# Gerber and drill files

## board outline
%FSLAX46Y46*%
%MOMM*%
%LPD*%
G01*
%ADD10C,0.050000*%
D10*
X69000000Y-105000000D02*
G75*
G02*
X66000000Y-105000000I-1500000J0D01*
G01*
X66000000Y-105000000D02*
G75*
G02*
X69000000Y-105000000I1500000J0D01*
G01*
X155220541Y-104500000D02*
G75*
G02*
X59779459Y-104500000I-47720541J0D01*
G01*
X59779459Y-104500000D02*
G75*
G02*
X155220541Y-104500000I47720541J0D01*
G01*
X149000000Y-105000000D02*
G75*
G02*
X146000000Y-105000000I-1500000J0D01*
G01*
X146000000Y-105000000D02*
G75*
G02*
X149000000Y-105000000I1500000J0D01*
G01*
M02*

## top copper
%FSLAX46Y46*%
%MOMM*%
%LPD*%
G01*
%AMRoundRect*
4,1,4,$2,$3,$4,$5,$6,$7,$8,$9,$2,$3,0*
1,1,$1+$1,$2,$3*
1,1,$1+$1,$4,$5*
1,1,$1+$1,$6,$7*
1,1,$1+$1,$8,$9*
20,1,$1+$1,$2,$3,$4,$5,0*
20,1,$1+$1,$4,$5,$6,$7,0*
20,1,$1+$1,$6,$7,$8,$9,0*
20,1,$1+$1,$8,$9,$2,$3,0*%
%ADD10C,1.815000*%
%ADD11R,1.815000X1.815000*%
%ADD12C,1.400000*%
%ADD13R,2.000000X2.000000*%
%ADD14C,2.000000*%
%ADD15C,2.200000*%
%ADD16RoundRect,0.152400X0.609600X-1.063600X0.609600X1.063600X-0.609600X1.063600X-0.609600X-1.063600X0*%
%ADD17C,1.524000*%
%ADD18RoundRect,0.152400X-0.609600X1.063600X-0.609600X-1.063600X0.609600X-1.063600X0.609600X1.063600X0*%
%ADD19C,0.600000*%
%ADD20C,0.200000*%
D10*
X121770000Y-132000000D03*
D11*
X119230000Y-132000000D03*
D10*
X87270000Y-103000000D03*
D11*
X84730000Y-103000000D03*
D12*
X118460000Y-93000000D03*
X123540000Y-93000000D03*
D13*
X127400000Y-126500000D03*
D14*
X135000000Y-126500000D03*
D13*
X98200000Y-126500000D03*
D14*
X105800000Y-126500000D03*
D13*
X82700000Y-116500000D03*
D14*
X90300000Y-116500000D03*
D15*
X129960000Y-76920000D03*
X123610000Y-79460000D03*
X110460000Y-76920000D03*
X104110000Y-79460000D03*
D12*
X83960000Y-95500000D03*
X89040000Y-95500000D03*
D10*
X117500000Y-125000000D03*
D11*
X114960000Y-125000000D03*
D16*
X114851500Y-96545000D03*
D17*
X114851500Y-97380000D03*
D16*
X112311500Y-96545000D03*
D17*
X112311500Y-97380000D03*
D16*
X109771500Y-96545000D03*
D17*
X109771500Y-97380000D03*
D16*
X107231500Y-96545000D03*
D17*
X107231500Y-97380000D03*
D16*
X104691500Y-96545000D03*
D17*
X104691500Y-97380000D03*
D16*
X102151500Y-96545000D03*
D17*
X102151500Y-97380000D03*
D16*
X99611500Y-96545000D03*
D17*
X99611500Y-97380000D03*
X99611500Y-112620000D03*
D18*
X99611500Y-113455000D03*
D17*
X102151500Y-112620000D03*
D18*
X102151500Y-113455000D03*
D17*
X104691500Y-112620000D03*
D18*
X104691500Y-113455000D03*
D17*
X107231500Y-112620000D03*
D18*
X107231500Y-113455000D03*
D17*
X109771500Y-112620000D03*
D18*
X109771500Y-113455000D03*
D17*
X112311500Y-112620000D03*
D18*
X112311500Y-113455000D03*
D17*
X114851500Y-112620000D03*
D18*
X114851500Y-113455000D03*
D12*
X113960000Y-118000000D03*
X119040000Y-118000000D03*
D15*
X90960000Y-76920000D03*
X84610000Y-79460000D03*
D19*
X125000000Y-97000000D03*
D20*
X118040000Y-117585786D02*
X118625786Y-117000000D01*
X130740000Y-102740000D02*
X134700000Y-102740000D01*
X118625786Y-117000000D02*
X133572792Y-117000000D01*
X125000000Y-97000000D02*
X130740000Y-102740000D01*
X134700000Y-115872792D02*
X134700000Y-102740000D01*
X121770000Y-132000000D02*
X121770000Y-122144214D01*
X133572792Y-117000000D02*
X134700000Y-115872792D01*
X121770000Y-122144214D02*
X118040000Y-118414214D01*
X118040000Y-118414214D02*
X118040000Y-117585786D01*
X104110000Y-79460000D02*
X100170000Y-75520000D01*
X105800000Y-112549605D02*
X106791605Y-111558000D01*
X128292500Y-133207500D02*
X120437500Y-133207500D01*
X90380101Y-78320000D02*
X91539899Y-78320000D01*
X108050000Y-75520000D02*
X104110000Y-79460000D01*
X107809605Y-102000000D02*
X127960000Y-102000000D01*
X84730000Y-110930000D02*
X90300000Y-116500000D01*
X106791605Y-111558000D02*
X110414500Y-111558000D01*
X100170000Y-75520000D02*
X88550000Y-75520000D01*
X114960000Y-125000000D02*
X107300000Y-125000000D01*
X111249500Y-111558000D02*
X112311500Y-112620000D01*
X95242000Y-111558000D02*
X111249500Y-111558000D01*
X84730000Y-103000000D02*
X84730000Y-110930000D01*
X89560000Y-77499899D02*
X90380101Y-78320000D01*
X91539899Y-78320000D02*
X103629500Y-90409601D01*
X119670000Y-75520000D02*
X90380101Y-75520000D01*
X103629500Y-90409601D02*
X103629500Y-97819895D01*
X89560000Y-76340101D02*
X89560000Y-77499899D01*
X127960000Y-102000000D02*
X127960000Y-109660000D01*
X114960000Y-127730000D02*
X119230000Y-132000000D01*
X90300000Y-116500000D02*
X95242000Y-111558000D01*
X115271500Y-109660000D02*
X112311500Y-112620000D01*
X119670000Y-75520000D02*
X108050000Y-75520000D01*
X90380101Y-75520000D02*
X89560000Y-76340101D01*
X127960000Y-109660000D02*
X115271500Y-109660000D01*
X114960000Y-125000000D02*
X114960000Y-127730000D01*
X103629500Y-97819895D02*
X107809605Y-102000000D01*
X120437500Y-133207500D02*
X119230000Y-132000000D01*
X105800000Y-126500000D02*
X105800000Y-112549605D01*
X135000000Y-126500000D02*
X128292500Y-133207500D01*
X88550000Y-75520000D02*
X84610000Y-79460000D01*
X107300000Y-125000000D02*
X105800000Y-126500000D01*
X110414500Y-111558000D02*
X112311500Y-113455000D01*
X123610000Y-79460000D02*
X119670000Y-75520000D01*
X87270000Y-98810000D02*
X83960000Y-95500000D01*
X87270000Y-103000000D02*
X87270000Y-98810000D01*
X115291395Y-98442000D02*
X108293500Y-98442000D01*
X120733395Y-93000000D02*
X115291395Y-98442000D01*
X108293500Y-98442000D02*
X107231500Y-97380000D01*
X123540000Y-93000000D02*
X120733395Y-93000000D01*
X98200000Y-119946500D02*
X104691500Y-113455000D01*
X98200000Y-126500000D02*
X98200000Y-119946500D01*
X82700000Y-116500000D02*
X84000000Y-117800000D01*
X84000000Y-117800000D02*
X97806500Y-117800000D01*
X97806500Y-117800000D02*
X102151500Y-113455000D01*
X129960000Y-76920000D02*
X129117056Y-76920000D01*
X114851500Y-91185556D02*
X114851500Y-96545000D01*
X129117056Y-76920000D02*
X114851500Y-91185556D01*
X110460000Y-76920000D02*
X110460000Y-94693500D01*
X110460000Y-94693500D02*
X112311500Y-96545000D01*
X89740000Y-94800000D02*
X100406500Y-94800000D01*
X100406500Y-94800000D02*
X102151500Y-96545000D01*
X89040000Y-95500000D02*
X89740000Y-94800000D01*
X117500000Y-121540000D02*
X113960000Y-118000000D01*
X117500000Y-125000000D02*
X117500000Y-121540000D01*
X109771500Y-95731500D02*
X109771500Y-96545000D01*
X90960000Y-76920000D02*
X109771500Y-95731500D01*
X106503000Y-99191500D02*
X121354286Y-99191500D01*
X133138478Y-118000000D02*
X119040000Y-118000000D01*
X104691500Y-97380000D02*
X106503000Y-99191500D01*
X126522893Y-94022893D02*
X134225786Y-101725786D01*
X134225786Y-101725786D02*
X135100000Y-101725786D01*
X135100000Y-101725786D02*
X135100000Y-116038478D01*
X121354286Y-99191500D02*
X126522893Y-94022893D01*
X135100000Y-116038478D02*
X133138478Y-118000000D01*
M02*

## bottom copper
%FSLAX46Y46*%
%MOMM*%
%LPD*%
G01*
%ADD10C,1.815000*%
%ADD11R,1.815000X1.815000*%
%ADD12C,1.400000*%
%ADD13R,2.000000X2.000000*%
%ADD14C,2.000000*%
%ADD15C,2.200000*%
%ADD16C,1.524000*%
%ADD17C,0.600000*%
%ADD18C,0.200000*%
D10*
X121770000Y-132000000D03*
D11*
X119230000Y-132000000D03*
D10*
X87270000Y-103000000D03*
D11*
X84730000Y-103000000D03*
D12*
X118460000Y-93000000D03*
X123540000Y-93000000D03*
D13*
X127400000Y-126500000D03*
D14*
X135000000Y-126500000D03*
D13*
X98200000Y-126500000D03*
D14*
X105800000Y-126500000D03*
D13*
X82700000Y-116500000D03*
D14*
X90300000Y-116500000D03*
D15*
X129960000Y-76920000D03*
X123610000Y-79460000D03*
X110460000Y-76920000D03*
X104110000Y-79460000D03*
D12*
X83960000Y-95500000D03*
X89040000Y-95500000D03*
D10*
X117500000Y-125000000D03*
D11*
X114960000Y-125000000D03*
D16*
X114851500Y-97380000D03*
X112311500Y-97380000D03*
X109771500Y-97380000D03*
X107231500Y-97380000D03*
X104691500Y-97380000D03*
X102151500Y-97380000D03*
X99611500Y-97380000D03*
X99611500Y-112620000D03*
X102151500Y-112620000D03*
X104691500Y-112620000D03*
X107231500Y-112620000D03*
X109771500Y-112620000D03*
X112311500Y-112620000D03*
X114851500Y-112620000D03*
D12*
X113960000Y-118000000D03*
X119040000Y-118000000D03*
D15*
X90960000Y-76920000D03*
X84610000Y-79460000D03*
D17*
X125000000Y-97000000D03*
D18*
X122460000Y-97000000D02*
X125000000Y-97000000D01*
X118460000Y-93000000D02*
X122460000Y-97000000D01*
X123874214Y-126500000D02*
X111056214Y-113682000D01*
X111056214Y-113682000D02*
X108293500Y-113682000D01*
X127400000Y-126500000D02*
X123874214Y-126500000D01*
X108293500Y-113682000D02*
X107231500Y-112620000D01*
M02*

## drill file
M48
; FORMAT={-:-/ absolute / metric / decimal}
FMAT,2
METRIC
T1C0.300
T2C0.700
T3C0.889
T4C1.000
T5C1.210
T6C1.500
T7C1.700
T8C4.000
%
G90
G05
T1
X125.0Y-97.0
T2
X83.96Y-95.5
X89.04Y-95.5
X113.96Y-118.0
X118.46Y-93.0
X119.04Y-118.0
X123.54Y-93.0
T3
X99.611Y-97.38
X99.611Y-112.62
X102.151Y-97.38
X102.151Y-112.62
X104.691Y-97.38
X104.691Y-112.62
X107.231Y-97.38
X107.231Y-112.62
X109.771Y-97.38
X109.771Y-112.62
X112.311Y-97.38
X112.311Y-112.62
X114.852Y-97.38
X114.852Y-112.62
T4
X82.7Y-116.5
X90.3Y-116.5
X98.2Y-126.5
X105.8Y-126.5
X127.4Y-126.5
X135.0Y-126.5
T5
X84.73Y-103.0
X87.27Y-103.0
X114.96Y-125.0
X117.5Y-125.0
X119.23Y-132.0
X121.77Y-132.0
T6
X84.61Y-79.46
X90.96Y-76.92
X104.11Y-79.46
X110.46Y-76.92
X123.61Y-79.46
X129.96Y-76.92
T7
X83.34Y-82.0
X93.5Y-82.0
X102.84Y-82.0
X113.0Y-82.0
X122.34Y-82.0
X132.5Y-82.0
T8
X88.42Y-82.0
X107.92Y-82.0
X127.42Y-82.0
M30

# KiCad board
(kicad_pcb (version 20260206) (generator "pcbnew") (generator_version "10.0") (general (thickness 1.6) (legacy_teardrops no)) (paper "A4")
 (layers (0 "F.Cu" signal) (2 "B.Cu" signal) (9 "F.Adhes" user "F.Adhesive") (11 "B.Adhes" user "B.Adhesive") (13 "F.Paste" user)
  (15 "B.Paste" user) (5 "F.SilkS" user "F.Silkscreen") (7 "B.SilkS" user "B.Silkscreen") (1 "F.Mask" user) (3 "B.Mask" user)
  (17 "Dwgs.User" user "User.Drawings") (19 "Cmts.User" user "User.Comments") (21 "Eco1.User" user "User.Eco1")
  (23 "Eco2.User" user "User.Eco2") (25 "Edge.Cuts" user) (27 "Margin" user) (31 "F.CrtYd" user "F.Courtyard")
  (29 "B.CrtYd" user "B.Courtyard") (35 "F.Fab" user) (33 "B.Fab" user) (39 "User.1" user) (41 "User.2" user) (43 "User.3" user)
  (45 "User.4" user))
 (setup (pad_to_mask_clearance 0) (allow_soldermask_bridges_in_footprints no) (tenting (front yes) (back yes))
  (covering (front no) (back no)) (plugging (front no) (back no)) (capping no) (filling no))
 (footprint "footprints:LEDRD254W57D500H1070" (layer "F.Cu") (at 120.5 132)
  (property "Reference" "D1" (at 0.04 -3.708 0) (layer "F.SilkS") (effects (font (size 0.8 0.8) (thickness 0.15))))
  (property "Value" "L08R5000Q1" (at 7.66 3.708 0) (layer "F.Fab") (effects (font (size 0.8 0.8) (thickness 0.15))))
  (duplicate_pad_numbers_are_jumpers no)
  (pad "A" thru_hole circle (at 1.27 0) (size 1.815 1.815) (drill 1.21) (layers "*.Cu" "*.Mask") (remove_unused_layers no)
   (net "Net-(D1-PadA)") (solder_mask_margin 0.102))
  (pad "C" thru_hole rect (at -1.27 0) (size 1.815 1.815) (drill 1.21) (layers "*.Cu" "*.Mask") (remove_unused_layers no) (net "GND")
   (solder_mask_margin 0.102)))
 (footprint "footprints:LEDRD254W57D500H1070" (layer "F.Cu") (at 86 103)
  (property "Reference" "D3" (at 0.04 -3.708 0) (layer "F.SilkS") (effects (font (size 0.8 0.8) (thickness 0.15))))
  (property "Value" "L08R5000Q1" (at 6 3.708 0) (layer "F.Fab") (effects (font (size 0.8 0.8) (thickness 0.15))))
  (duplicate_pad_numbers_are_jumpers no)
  (pad "A" thru_hole circle (at 1.27 0) (size 1.815 1.815) (drill 1.21) (layers "*.Cu" "*.Mask") (remove_unused_layers no)
   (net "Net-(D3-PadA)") (solder_mask_margin 0.102))
  (pad "C" thru_hole rect (at -1.27 0) (size 1.815 1.815) (drill 1.21) (layers "*.Cu" "*.Mask") (remove_unused_layers no) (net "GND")
   (solder_mask_margin 0.102)))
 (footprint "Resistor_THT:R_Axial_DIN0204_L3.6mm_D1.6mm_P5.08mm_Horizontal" (layer "F.Cu") (at 118.46 93)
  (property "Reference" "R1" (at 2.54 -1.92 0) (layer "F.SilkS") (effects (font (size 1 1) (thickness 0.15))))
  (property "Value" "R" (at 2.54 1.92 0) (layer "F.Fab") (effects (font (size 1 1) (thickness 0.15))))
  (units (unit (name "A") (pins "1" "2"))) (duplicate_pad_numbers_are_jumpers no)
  (pad "1" thru_hole circle (at 0 0) (size 1.4 1.4) (drill 0.7) (layers "*.Cu" "*.Mask") (remove_unused_layers no) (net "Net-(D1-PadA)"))
  (pad "2" thru_hole circle (at 5.08 0) (size 1.4 1.4) (drill 0.7) (layers "*.Cu" "*.Mask") (remove_unused_layers no)
   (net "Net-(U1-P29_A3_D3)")))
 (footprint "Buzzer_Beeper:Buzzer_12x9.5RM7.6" (layer "F.Cu") (at 127.4 126.5)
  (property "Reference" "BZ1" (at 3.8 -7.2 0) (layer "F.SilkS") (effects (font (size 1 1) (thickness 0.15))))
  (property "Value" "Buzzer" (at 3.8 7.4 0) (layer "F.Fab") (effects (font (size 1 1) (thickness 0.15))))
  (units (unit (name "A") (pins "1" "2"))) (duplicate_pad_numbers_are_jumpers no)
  (pad "1" thru_hole rect (at 0 0) (size 2 2) (drill 1) (layers "*.Cu" "*.Mask") (remove_unused_layers no) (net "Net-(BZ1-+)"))
  (pad "2" thru_hole circle (at 7.6 0) (size 2 2) (drill 1) (layers "*.Cu" "*.Mask") (remove_unused_layers no) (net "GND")))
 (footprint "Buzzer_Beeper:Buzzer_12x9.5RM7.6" (layer "F.Cu") (at 98.2 126.5)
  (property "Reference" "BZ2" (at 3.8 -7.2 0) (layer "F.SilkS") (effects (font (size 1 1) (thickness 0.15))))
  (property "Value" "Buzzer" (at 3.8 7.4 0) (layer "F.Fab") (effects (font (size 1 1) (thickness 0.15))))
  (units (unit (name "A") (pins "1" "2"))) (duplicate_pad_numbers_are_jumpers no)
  (pad "1" thru_hole rect (at 0 0) (size 2 2) (drill 1) (layers "*.Cu" "*.Mask") (remove_unused_layers no) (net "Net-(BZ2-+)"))
  (pad "2" thru_hole circle (at 7.6 0) (size 2 2) (drill 1) (layers "*.Cu" "*.Mask") (remove_unused_layers no) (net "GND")))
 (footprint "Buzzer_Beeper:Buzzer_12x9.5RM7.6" (layer "F.Cu") (at 82.7 116.5)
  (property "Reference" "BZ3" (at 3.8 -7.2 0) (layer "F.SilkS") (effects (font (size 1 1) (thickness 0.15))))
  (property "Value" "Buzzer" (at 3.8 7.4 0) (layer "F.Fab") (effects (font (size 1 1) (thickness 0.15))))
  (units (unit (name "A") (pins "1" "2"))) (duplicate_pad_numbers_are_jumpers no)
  (pad "1" thru_hole rect (at 0 0) (size 2 2) (drill 1) (layers "*.Cu" "*.Mask") (remove_unused_layers no) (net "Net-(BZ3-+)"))
  (pad "2" thru_hole circle (at 7.6 0) (size 2 2) (drill 1) (layers "*.Cu" "*.Mask") (remove_unused_layers no) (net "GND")))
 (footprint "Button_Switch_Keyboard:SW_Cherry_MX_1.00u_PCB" (layer "F.Cu") (at 129.96 76.92)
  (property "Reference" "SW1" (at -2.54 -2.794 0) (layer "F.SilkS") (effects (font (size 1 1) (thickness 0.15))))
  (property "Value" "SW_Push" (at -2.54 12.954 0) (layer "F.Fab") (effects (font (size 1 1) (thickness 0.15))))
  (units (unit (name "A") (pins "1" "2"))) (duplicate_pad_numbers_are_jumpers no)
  (pad "" np_thru_hole circle (at -7.62 5.08) (size 1.7 1.7) (drill 1.7) (layers "*.Cu" "*.Mask"))
  (pad "" np_thru_hole circle (at -2.54 5.08) (size 4 4) (drill 4) (layers "*.Cu" "*.Mask"))
  (pad "" np_thru_hole circle (at 2.54 5.08) (size 1.7 1.7) (drill 1.7) (layers "*.Cu" "*.Mask"))
  (pad "1" thru_hole circle (at 0 0) (size 2.2 2.2) (drill 1.5) (layers "*.Cu" "*.Mask") (remove_unused_layers no)
   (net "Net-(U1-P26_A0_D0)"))
  (pad "2" thru_hole circle (at -6.35 2.54) (size 2.2 2.2) (drill 1.5) (layers "*.Cu" "*.Mask") (remove_unused_layers no) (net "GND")))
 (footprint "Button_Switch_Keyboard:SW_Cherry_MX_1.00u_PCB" (layer "F.Cu") (at 110.46 76.92)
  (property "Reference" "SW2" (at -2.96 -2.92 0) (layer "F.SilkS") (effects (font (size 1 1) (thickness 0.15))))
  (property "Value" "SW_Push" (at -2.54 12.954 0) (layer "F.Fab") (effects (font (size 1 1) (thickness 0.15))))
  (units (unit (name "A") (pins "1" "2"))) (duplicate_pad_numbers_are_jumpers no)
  (pad "" np_thru_hole circle (at -7.62 5.08) (size 1.7 1.7) (drill 1.7) (layers "*.Cu" "*.Mask"))
  (pad "" np_thru_hole circle (at -2.54 5.08) (size 4 4) (drill 4) (layers "*.Cu" "*.Mask"))
  (pad "" np_thru_hole circle (at 2.54 5.08) (size 1.7 1.7) (drill 1.7) (layers "*.Cu" "*.Mask"))
  (pad "1" thru_hole circle (at 0 0) (size 2.2 2.2) (drill 1.5) (layers "*.Cu" "*.Mask") (remove_unused_layers no)
   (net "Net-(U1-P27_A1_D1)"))
  (pad "2" thru_hole circle (at -6.35 2.54) (size 2.2 2.2) (drill 1.5) (layers "*.Cu" "*.Mask") (remove_unused_layers no) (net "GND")))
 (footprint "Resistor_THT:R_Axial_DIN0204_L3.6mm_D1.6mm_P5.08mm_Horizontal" (layer "F.Cu") (at 83.96 95.5)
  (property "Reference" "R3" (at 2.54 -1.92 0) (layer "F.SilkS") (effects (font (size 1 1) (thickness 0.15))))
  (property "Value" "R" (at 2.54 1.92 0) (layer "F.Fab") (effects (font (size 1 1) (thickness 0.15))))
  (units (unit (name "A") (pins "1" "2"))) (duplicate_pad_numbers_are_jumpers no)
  (pad "1" thru_hole circle (at 0 0) (size 1.4 1.4) (drill 0.7) (layers "*.Cu" "*.Mask") (remove_unused_layers no) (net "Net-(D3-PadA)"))
  (pad "2" thru_hole circle (at 5.08 0) (size 1.4 1.4) (drill 0.7) (layers "*.Cu" "*.Mask") (remove_unused_layers no)
   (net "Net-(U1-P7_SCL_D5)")))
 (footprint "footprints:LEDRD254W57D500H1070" (layer "F.Cu") (at 116.23 125)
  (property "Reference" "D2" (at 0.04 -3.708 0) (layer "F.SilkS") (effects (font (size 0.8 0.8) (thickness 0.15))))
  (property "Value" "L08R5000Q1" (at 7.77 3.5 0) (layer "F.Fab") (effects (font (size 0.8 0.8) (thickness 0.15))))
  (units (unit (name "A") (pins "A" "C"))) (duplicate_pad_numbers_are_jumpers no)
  (pad "A" thru_hole circle (at 1.27 0) (size 1.815 1.815) (drill 1.21) (layers "*.Cu" "*.Mask") (remove_unused_layers no)
   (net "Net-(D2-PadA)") (solder_mask_margin 0.102))
  (pad "C" thru_hole rect (at -1.27 0) (size 1.815 1.815) (drill 1.21) (layers "*.Cu" "*.Mask") (remove_unused_layers no) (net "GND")
   (solder_mask_margin 0.102)))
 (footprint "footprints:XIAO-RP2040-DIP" (layer "F.Cu") (at 107.2315 105)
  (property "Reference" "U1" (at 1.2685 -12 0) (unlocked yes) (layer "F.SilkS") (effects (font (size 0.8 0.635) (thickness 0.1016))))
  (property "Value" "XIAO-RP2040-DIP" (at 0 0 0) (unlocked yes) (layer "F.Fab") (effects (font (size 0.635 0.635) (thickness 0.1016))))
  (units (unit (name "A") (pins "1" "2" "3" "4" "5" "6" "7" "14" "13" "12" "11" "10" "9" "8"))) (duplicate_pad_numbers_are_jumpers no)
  (pad "1" smd roundrect (at 7.62 -8.455 90) (size 2.432 1.524) (layers "F.Cu" "F.Mask") (roundrect_rratio 0.1) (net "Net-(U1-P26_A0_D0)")
   (thermal_bridge_angle 45))
  (pad "1" thru_hole circle (at 7.62 -7.62 90) (size 1.524 1.524) (drill 0.889) (layers "*.Cu" "*.Mask") (remove_unused_layers no)
   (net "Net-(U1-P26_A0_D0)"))
  (pad "2" smd roundrect (at 5.08 -8.455 90) (size 2.432 1.524) (layers "F.Cu" "F.Mask") (roundrect_rratio 0.1) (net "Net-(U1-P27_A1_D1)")
   (thermal_bridge_angle 45))
  (pad "2" thru_hole circle (at 5.08 -7.62 90) (size 1.524 1.524) (drill 0.889) (layers "*.Cu" "*.Mask") (remove_unused_layers no)
   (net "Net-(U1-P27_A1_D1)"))
  (pad "3" smd roundrect (at 2.54 -8.455 90) (size 2.432 1.524) (layers "F.Cu" "F.Mask") (roundrect_rratio 0.1) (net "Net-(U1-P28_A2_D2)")
   (thermal_bridge_angle 45))
  (pad "3" thru_hole circle (at 2.54 -7.62 90) (size 1.524 1.524) (drill 0.889) (layers "*.Cu" "*.Mask") (remove_unused_layers no)
   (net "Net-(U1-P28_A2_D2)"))
  (pad "4" smd roundrect (at 0 -8.455 90) (size 2.432 1.524) (layers "F.Cu" "F.Mask") (roundrect_rratio 0.1) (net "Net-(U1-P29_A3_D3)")
   (thermal_bridge_angle 45))
  (pad "4" thru_hole circle (at 0 -7.62 90) (size 1.524 1.524) (drill 0.889) (layers "*.Cu" "*.Mask") (remove_unused_layers no)
   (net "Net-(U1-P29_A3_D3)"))
  (pad "5" smd roundrect (at -2.54 -8.455 90) (size 2.432 1.524) (layers "F.Cu" "F.Mask") (roundrect_rratio 0.1) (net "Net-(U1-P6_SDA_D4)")
   (thermal_bridge_angle 45))
  (pad "5" thru_hole circle (at -2.54 -7.62 90) (size 1.524 1.524) (drill 0.889) (layers "*.Cu" "*.Mask") (remove_unused_layers no)
   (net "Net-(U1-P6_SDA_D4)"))
  (pad "6" smd roundrect (at -5.08 -8.455 90) (size 2.432 1.524) (layers "F.Cu" "F.Mask") (roundrect_rratio 0.1) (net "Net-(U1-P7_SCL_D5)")
   (thermal_bridge_angle 45))
  (pad "6" thru_hole circle (at -5.08 -7.62 90) (size 1.524 1.524) (drill 0.889) (layers "*.Cu" "*.Mask") (remove_unused_layers no)
   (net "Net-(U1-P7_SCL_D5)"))
  (pad "7" smd roundrect (at -7.62 -8.455 90) (size 2.432 1.524) (layers "F.Cu" "F.Mask") (roundrect_rratio 0.1)
   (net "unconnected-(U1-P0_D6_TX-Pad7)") (thermal_bridge_angle 45))
  (pad "7" thru_hole circle (at -7.62 -7.62 90) (size 1.524 1.524) (drill 0.889) (layers "*.Cu" "*.Mask") (remove_unused_layers no)
   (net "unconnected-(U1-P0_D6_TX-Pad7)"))
  (pad "8" thru_hole circle (at -7.62 7.62 270) (size 1.524 1.524) (drill 0.889) (layers "*.Cu" "*.Mask") (remove_unused_layers no)
   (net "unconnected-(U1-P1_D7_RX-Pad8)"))
  (pad "8" smd roundrect (at -7.62 8.455 270) (size 2.432 1.524) (layers "F.Cu" "F.Mask") (roundrect_rratio 0.1)
   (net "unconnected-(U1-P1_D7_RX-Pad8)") (thermal_bridge_angle 45))
  (pad "9" thru_hole circle (at -5.08 7.62 270) (size 1.524 1.524) (drill 0.889) (layers "*.Cu" "*.Mask") (remove_unused_layers no)
   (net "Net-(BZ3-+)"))
  (pad "9" smd roundrect (at -5.08 8.455 270) (size 2.432 1.524) (layers "F.Cu" "F.Mask") (roundrect_rratio 0.1) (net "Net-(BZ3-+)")
   (thermal_bridge_angle 45))
  (pad "10" thru_hole circle (at -2.54 7.62 270) (size 1.524 1.524) (drill 0.889) (layers "*.Cu" "*.Mask") (remove_unused_layers no)
   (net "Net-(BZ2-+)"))
  (pad "10" smd roundrect (at -2.54 8.455 270) (size 2.432 1.524) (layers "F.Cu" "F.Mask") (roundrect_rratio 0.1) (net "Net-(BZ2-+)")
   (thermal_bridge_angle 45))
  (pad "11" thru_hole circle (at 0 7.62 270) (size 1.524 1.524) (drill 0.889) (layers "*.Cu" "*.Mask") (remove_unused_layers no)
   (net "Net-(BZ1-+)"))
  (pad "11" smd roundrect (at 0 8.455 270) (size 2.432 1.524) (layers "F.Cu" "F.Mask") (roundrect_rratio 0.1) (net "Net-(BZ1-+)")
   (thermal_bridge_angle 45))
  (pad "12" thru_hole circle (at 2.54 7.62 270) (size 1.524 1.524) (drill 0.889) (layers "*.Cu" "*.Mask") (remove_unused_layers no)
   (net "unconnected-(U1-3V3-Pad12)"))
  (pad "12" smd roundrect (at 2.54 8.455 270) (size 2.432 1.524) (layers "F.Cu" "F.Mask") (roundrect_rratio 0.1)
   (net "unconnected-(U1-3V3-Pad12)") (thermal_bridge_angle 45))
  (pad "13" thru_hole circle (at 5.08 7.62 270) (size 1.524 1.524) (drill 0.889) (layers "*.Cu" "*.Mask") (remove_unused_layers no)
   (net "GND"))
  (pad "13" smd roundrect (at 5.08 8.455 270) (size 2.432 1.524) (layers "F.Cu" "F.Mask") (roundrect_rratio 0.1) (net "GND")
   (thermal_bridge_angle 45))
  (pad "14" thru_hole circle (at 7.62 7.62 270) (size 1.524 1.524) (drill 0.889) (layers "*.Cu" "*.Mask") (remove_unused_layers no)
   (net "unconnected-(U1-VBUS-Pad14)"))
  (pad "14" smd roundrect (at 7.62 8.455 270) (size 2.432 1.524) (layers "F.Cu" "F.Mask") (roundrect_rratio 0.1)
   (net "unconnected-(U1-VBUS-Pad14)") (thermal_bridge_angle 45)))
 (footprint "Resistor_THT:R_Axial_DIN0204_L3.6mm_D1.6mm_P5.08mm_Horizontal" (layer "F.Cu") (at 113.96 118)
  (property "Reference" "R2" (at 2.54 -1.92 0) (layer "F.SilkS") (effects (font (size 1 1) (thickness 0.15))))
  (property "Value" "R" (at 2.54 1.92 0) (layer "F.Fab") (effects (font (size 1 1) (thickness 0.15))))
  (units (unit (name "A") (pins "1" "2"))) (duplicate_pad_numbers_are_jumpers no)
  (pad "1" thru_hole circle (at 0 0) (size 1.4 1.4) (drill 0.7) (layers "*.Cu" "*.Mask") (remove_unused_layers no) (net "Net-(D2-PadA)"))
  (pad "2" thru_hole circle (at 5.08 0) (size 1.4 1.4) (drill 0.7) (layers "*.Cu" "*.Mask") (remove_unused_layers no)
   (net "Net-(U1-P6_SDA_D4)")))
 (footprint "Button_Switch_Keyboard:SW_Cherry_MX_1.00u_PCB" (layer "F.Cu") (at 90.96 76.92)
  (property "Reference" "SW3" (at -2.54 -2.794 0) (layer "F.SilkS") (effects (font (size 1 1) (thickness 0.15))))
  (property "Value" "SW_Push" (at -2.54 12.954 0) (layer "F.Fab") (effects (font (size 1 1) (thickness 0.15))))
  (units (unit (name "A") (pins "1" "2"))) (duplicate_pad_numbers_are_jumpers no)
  (pad "" np_thru_hole circle (at -7.62 5.08) (size 1.7 1.7) (drill 1.7) (layers "*.Cu" "*.Mask"))
  (pad "" np_thru_hole circle (at -2.54 5.08) (size 4 4) (drill 4) (layers "*.Cu" "*.Mask"))
  (pad "" np_thru_hole circle (at 2.54 5.08) (size 1.7 1.7) (drill 1.7) (layers "*.Cu" "*.Mask"))
  (pad "1" thru_hole circle (at 0 0) (size 2.2 2.2) (drill 1.5) (layers "*.Cu" "*.Mask") (remove_unused_layers no)
   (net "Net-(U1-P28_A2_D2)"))
  (pad "2" thru_hole circle (at -6.35 2.54) (size 2.2 2.2) (drill 1.5) (layers "*.Cu" "*.Mask") (remove_unused_layers no) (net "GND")))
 (gr_circle (center 67.5 105) (end 66 105) (stroke (width 0.05) (type default)) (fill no) (layer "Edge.Cuts"))
 (gr_circle (center 107.5 104.5) (end 80 65.5) (stroke (width 0.05) (type default)) (fill no) (layer "Edge.Cuts"))
 (gr_circle (center 147.5 105) (end 149 105) (stroke (width 0.05) (type default)) (fill no) (layer "Edge.Cuts"))
 (segment (start 118.04 117.585786) (end 118.625786 117) (width 0.2) (layer "F.Cu") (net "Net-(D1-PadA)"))
 (segment (start 130.74 102.74) (end 134.7 102.74) (width 0.2) (layer "F.Cu") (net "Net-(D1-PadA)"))
 (segment (start 118.625786 117) (end 133.572792 117) (width 0.2) (layer "F.Cu") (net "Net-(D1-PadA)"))
 (segment (start 125 97) (end 130.74 102.74) (width 0.2) (layer "F.Cu") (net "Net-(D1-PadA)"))
 (segment (start 134.7 115.872792) (end 134.7 102.74) (width 0.2) (layer "F.Cu") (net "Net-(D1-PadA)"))
 (segment (start 121.77 132) (end 121.77 122.144214) (width 0.2) (layer "F.Cu") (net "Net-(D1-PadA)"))
 (segment (start 133.572792 117) (end 134.7 115.872792) (width 0.2) (layer "F.Cu") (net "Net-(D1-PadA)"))
 (segment (start 121.77 122.144214) (end 118.04 118.414214) (width 0.2) (layer "F.Cu") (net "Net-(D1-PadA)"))
 (segment (start 118.04 118.414214) (end 118.04 117.585786) (width 0.2) (layer "F.Cu") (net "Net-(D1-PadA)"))
 (via (at 125 97) (size 0.6) (drill 0.3) (layers "F.Cu" "B.Cu") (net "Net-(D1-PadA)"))
 (segment (start 122.46 97) (end 125 97) (width 0.2) (layer "B.Cu") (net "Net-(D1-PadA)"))
 (segment (start 118.46 93) (end 122.46 97) (width 0.2) (layer "B.Cu") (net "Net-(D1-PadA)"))
 (segment (start 104.11 79.46) (end 100.17 75.52) (width 0.2) (layer "F.Cu") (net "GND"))
 (segment (start 105.8 112.549605) (end 106.791605 111.558) (width 0.2) (layer "F.Cu") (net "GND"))
 (segment (start 128.2925 133.2075) (end 120.4375 133.2075) (width 0.2) (layer "F.Cu") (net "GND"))
 (segment (start 90.380101 78.32) (end 91.539899 78.32) (width 0.2) (layer "F.Cu") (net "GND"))
 (segment (start 108.05 75.52) (end 104.11 79.46) (width 0.2) (layer "F.Cu") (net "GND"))
 (segment (start 107.809605 102) (end 127.96 102) (width 0.2) (layer "F.Cu") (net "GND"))
 (segment (start 84.73 110.93) (end 90.3 116.5) (width 0.2) (layer "F.Cu") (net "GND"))
 (segment (start 106.791605 111.558) (end 110.4145 111.558) (width 0.2) (layer "F.Cu") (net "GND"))
 (segment (start 100.17 75.52) (end 88.55 75.52) (width 0.2) (layer "F.Cu") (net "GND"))
 (segment (start 114.96 125) (end 107.3 125) (width 0.2) (layer "F.Cu") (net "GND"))
 (segment (start 111.2495 111.558) (end 112.3115 112.62) (width 0.2) (layer "F.Cu") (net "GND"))
 (segment (start 95.242 111.558) (end 111.2495 111.558) (width 0.2) (layer "F.Cu") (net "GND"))
 (segment (start 84.73 103) (end 84.73 110.93) (width 0.2) (layer "F.Cu") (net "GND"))
 (segment (start 89.56 77.499899) (end 90.380101 78.32) (width 0.2) (layer "F.Cu") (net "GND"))
 (segment (start 91.539899 78.32) (end 103.6295 90.409601) (width 0.2) (layer "F.Cu") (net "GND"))
 (segment (start 119.67 75.52) (end 90.380101 75.52) (width 0.2) (layer "F.Cu") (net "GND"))
 (segment (start 103.6295 90.409601) (end 103.6295 97.819895) (width 0.2) (layer "F.Cu") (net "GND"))
 (segment (start 89.56 76.340101) (end 89.56 77.499899) (width 0.2) (layer "F.Cu") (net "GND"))
 (segment (start 127.96 102) (end 127.96 109.66) (width 0.2) (layer "F.Cu") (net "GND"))
 (segment (start 114.96 127.73) (end 119.23 132) (width 0.2) (layer "F.Cu") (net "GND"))
 (segment (start 90.3 116.5) (end 95.242 111.558) (width 0.2) (layer "F.Cu") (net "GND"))
 (segment (start 115.2715 109.66) (end 112.3115 112.62) (width 0.2) (layer "F.Cu") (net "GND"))
 (segment (start 119.67 75.52) (end 108.05 75.52) (width 0.2) (layer "F.Cu") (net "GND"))
 (segment (start 90.380101 75.52) (end 89.56 76.340101) (width 0.2) (layer "F.Cu") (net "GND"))
 (segment (start 127.96 109.66) (end 115.2715 109.66) (width 0.2) (layer "F.Cu") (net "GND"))
 (segment (start 114.96 125) (end 114.96 127.73) (width 0.2) (layer "F.Cu") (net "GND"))
 (segment (start 103.6295 97.819895) (end 107.809605 102) (width 0.2) (layer "F.Cu") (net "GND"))
 (segment (start 120.4375 133.2075) (end 119.23 132) (width 0.2) (layer "F.Cu") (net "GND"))
 (segment (start 105.8 126.5) (end 105.8 112.549605) (width 0.2) (layer "F.Cu") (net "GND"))
 (segment (start 135 126.5) (end 128.2925 133.2075) (width 0.2) (layer "F.Cu") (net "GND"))
 (segment (start 88.55 75.52) (end 84.61 79.46) (width 0.2) (layer "F.Cu") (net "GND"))
 (segment (start 107.3 125) (end 105.8 126.5) (width 0.2) (layer "F.Cu") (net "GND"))
 (segment (start 110.4145 111.558) (end 112.3115 113.455) (width 0.2) (layer "F.Cu") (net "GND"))
 (segment (start 123.61 79.46) (end 119.67 75.52) (width 0.2) (layer "F.Cu") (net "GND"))
 (segment (start 87.27 98.81) (end 83.96 95.5) (width 0.2) (layer "F.Cu") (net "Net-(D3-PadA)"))
 (segment (start 87.27 103) (end 87.27 98.81) (width 0.2) (layer "F.Cu") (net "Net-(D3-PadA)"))
 (segment (start 115.291395 98.442) (end 108.2935 98.442) (width 0.2) (layer "F.Cu") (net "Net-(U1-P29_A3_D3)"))
 (segment (start 120.733395 93) (end 115.291395 98.442) (width 0.2) (layer "F.Cu") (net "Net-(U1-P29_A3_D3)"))
 (segment (start 108.2935 98.442) (end 107.2315 97.38) (width 0.2) (layer "F.Cu") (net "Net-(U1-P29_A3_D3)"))
 (segment (start 123.54 93) (end 120.733395 93) (width 0.2) (layer "F.Cu") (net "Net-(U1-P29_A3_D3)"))
 (segment (start 123.874214 126.5) (end 111.056214 113.682) (width 0.2) (layer "B.Cu") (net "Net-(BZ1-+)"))
 (segment (start 111.056214 113.682) (end 108.2935 113.682) (width 0.2) (layer "B.Cu") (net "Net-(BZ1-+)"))
 (segment (start 127.4 126.5) (end 123.874214 126.5) (width 0.2) (layer "B.Cu") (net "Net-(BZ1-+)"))
 (segment (start 108.2935 113.682) (end 107.2315 112.62) (width 0.2) (layer "B.Cu") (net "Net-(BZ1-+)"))
 (segment (start 98.2 119.9465) (end 104.6915 113.455) (width 0.2) (layer "F.Cu") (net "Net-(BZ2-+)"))
 (segment (start 98.2 126.5) (end 98.2 119.9465) (width 0.2) (layer "F.Cu") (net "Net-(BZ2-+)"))
 (segment (start 82.7 116.5) (end 84 117.8) (width 0.2) (layer "F.Cu") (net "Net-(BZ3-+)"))
 (segment (start 84 117.8) (end 97.8065 117.8) (width 0.2) (layer "F.Cu") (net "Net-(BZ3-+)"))
 (segment (start 97.8065 117.8) (end 102.1515 113.455) (width 0.2) (layer "F.Cu") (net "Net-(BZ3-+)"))
 (segment (start 129.96 76.92) (end 129.117056 76.92) (width 0.2) (layer "F.Cu") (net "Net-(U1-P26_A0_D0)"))
 (segment (start 114.8515 91.185556) (end 114.8515 96.545) (width 0.2) (layer "F.Cu") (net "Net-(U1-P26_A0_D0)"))
 (segment (start 129.117056 76.92) (end 114.8515 91.185556) (width 0.2) (layer "F.Cu") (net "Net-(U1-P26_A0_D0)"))
 (segment (start 110.46 76.92) (end 110.46 94.6935) (width 0.2) (layer "F.Cu") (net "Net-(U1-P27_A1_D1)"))
 (segment (start 110.46 94.6935) (end 112.3115 96.545) (width 0.2) (layer "F.Cu") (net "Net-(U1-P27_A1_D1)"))
 (segment (start 89.74 94.8) (end 100.4065 94.8) (width 0.2) (layer "F.Cu") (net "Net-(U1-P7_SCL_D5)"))
 (segment (start 100.4065 94.8) (end 102.1515 96.545) (width 0.2) (layer "F.Cu") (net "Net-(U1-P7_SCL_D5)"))
 (segment (start 89.04 95.5) (end 89.74 94.8) (width 0.2) (layer "F.Cu") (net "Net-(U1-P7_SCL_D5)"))
 (segment (start 117.5 121.54) (end 113.96 118) (width 0.2) (layer "F.Cu") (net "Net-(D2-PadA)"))
 (segment (start 117.5 125) (end 117.5 121.54) (width 0.2) (layer "F.Cu") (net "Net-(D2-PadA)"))
 (segment (start 109.7715 95.7315) (end 109.7715 96.545) (width 0.2) (layer "F.Cu") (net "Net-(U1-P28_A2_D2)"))
 (segment (start 90.96 76.92) (end 109.7715 95.7315) (width 0.2) (layer "F.Cu") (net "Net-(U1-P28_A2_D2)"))
 (segment (start 106.503 99.1915) (end 121.354286 99.1915) (width 0.2) (layer "F.Cu") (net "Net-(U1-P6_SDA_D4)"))
 (segment (start 133.138478 118) (end 119.04 118) (width 0.2) (layer "F.Cu") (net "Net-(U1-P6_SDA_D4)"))
 (segment (start 104.6915 97.38) (end 106.503 99.1915) (width 0.2) (layer "F.Cu") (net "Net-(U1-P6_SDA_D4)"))
 (segment (start 126.522893 94.022893) (end 134.225786 101.725786) (width 0.2) (layer "F.Cu") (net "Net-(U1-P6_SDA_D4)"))
 (segment (start 134.225786 101.725786) (end 135.1 101.725786) (width 0.2) (layer "F.Cu") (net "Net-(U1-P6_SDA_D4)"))
 (segment (start 135.1 101.725786) (end 135.1 116.038478) (width 0.2) (layer "F.Cu") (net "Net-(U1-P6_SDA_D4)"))
 (segment (start 121.354286 99.1915) (end 126.522893 94.022893) (width 0.2) (layer "F.Cu") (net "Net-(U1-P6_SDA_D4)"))
 (segment (start 135.1 116.038478) (end 133.138478 118) (width 0.2) (layer "F.Cu") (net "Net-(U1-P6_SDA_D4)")))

